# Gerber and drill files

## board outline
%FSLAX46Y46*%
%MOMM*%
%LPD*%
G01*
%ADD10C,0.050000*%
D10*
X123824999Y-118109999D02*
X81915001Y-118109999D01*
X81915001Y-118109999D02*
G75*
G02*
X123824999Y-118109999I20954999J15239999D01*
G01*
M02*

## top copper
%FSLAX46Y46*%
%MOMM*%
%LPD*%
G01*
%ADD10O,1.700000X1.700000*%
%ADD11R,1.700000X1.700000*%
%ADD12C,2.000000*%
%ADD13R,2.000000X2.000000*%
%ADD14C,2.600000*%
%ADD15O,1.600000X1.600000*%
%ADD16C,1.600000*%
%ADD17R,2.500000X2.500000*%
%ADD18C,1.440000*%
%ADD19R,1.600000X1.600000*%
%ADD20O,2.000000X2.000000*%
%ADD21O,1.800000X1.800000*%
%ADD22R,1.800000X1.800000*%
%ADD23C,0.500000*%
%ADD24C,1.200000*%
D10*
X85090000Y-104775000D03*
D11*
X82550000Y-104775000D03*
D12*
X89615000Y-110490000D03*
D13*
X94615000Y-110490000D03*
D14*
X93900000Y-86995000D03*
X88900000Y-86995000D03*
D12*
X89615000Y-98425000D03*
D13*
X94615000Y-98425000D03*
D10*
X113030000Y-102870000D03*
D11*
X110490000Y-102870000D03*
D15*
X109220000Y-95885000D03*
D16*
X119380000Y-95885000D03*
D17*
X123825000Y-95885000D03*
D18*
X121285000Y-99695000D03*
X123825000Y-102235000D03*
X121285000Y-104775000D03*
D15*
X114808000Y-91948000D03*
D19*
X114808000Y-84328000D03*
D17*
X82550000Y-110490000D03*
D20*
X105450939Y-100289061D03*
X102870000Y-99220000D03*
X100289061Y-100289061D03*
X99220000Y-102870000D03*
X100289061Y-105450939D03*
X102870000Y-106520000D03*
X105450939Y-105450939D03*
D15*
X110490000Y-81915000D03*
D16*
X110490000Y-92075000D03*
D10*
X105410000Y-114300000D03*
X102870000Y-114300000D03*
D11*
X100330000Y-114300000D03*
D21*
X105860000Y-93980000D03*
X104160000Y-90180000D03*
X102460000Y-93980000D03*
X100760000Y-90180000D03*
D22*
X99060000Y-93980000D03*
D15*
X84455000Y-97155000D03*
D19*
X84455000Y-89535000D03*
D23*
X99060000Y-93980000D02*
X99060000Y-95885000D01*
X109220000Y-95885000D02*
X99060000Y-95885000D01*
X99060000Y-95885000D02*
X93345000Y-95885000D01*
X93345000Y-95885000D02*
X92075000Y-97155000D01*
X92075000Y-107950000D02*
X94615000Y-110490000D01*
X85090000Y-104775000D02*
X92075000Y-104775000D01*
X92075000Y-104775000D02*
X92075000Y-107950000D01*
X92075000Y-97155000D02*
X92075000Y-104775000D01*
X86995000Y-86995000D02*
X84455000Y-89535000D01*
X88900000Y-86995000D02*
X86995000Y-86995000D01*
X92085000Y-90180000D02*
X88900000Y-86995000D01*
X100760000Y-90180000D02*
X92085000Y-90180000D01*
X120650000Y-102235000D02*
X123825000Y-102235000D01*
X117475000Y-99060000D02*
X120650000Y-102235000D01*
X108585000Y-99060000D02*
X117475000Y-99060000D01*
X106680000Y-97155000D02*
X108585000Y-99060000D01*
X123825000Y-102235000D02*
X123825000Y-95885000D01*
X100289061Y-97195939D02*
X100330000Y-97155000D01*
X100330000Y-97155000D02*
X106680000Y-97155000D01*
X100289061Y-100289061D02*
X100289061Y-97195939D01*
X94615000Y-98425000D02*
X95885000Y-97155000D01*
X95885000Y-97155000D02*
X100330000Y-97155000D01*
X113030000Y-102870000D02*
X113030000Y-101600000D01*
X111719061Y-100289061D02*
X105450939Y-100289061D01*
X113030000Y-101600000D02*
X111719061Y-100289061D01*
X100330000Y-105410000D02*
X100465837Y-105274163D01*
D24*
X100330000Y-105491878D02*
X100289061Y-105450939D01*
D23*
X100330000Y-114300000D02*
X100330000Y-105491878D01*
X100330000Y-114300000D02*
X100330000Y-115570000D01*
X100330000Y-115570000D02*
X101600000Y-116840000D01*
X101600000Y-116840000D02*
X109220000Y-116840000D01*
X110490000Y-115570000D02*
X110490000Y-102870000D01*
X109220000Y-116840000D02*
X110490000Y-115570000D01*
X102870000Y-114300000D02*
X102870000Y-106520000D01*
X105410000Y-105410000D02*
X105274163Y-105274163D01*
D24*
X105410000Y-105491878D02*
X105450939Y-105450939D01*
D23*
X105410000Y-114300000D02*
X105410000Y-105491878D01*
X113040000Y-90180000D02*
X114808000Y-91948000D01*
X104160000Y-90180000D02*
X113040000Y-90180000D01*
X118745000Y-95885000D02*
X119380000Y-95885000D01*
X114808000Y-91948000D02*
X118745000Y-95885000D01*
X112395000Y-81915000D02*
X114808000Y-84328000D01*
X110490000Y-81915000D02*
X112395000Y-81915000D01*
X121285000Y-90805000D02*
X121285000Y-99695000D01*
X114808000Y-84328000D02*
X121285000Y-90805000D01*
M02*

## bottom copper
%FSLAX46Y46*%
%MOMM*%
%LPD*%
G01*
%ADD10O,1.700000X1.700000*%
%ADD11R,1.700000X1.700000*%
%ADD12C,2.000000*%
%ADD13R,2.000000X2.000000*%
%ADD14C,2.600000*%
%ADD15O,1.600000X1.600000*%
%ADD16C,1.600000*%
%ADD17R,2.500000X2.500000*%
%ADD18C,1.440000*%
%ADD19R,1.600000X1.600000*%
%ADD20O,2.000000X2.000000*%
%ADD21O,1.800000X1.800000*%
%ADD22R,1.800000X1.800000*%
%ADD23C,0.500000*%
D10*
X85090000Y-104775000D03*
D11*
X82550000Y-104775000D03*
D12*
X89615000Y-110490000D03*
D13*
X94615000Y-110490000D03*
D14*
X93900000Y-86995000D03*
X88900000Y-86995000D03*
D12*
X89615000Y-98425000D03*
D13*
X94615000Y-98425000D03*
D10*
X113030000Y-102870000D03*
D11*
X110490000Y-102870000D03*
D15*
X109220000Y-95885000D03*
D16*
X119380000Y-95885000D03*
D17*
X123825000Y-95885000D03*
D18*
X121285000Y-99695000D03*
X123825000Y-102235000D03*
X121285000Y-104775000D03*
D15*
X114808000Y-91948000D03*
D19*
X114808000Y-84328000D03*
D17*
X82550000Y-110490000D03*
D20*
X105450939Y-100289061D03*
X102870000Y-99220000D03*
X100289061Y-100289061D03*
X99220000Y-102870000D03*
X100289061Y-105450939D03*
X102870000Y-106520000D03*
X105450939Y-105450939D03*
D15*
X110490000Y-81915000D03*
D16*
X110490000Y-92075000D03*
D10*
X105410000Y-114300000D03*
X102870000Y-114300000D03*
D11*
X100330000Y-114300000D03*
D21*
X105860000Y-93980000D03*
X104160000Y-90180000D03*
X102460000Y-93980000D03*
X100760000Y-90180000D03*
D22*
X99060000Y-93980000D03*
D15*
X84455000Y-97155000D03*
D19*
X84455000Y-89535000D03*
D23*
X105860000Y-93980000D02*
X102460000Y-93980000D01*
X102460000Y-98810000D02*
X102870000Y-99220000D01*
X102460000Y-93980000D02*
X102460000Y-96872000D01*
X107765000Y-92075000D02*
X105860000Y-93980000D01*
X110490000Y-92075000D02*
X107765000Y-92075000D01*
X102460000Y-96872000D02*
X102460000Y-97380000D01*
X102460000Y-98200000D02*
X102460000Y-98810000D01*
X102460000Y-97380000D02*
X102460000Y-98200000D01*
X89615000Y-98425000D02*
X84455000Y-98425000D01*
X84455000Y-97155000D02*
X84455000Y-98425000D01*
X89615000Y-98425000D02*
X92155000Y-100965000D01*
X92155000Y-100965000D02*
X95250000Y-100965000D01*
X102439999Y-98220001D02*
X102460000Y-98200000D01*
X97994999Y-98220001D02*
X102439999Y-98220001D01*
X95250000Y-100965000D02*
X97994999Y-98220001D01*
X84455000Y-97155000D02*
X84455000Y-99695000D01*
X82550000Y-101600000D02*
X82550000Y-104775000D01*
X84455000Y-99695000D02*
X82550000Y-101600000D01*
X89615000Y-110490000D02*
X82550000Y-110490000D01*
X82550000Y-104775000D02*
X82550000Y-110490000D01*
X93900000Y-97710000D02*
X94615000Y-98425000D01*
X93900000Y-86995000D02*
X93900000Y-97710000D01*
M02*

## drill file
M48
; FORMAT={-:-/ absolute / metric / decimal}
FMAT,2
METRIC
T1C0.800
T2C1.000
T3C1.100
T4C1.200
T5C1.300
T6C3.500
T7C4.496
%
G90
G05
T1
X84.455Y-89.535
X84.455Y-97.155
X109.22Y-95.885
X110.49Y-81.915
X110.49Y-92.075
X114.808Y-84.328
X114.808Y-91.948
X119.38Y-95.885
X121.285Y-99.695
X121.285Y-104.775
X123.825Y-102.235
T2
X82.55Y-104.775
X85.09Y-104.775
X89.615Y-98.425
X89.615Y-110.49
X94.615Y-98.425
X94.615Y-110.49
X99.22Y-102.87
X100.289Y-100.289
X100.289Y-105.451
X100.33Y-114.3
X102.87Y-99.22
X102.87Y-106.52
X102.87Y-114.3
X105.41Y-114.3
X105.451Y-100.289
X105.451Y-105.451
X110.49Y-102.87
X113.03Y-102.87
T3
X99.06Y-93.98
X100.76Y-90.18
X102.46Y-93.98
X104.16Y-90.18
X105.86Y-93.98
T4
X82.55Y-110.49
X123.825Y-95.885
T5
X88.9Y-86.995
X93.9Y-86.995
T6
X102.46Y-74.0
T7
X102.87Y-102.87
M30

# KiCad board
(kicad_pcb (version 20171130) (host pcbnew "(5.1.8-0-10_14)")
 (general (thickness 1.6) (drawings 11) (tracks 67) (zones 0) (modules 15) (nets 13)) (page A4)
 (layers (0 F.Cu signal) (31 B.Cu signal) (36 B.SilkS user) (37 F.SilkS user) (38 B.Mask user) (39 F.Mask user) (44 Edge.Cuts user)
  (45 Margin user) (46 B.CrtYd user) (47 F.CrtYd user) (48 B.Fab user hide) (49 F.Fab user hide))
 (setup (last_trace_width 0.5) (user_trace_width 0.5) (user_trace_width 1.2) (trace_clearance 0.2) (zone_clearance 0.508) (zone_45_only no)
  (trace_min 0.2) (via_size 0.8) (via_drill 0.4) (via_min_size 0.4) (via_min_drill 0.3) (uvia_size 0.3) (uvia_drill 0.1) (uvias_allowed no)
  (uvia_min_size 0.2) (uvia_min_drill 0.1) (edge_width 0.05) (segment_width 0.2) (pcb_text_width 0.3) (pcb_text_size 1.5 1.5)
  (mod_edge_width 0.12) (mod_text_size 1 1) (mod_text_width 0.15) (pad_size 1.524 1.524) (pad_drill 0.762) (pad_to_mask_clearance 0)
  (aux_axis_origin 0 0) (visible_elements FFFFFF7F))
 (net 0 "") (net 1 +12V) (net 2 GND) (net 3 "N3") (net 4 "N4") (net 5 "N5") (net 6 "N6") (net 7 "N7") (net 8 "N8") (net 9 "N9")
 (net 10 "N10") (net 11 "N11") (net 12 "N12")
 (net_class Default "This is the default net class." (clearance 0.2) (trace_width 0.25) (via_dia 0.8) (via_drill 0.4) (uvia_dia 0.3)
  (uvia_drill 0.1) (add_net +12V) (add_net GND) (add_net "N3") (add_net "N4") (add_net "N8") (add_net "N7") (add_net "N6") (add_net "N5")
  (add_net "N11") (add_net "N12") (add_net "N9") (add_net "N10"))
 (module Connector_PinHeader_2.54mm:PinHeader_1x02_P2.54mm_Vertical (layer F.Cu) (at 82.55 104.775 90)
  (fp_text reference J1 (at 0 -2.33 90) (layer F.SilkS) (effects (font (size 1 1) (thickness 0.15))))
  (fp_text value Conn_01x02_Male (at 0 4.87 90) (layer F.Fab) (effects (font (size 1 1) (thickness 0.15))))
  (pad 2 thru_hole oval (at 0 2.54 90) (size 1.7 1.7) (drill 1) (layers *.Cu *.Mask) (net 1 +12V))
  (pad 1 thru_hole rect (at 0 0 90) (size 1.7 1.7) (drill 1) (layers *.Cu *.Mask) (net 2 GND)))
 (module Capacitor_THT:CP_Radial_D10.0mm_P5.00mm (layer F.Cu) (at 94.615 110.49 180)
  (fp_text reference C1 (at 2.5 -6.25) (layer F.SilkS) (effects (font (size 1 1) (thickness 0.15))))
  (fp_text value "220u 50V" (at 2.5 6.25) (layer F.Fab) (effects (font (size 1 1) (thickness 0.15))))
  (pad 2 thru_hole circle (at 5 0 180) (size 2 2) (drill 1) (layers *.Cu *.Mask) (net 2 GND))
  (pad 1 thru_hole rect (at 0 0 180) (size 2 2) (drill 1) (layers *.Cu *.Mask) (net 1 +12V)))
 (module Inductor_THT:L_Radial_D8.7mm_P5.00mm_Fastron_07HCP (layer F.Cu) (at 88.9 86.995)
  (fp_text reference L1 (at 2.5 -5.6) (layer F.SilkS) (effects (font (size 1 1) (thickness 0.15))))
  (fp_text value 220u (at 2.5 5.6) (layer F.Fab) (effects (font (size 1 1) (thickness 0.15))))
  (pad 2 thru_hole circle (at 5 0) (size 2.6 2.6) (drill 1.3) (layers *.Cu *.Mask) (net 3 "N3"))
  (pad 1 thru_hole circle (at 0 0) (size 2.6 2.6) (drill 1.3) (layers *.Cu *.Mask) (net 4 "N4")))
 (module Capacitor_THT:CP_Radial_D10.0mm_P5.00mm (layer F.Cu) (at 94.615 98.425 180)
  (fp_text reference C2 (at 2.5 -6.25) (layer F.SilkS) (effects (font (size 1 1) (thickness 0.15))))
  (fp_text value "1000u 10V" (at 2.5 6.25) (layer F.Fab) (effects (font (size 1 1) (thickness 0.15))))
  (pad 2 thru_hole circle (at 5 0 180) (size 2 2) (drill 1) (layers *.Cu *.Mask) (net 2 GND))
  (pad 1 thru_hole rect (at 0 0 180) (size 2 2) (drill 1) (layers *.Cu *.Mask) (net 3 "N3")))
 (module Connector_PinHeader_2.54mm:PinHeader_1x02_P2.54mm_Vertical (layer F.Cu) (at 110.49 102.87 90)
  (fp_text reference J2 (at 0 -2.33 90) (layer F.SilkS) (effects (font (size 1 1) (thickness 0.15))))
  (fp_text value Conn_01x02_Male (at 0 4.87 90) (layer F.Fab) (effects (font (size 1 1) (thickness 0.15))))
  (pad 2 thru_hole oval (at 0 2.54 90) (size 1.7 1.7) (drill 1) (layers *.Cu *.Mask) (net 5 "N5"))
  (pad 1 thru_hole rect (at 0 0 90) (size 1.7 1.7) (drill 1) (layers *.Cu *.Mask) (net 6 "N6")))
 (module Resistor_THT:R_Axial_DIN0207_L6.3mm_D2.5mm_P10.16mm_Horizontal (layer F.Cu) (at 119.38 95.885 180)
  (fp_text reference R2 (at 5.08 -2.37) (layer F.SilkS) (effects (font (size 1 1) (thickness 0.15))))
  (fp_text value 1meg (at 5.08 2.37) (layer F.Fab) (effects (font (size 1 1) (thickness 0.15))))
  (pad 2 thru_hole oval (at 10.16 0 180) (size 1.6 1.6) (drill 0.8) (layers *.Cu *.Mask) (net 1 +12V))
  (pad 1 thru_hole circle (at 0 0 180) (size 1.6 1.6) (drill 0.8) (layers *.Cu *.Mask) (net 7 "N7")))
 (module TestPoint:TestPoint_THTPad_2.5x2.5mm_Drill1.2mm (layer F.Cu) (at 123.825 95.885)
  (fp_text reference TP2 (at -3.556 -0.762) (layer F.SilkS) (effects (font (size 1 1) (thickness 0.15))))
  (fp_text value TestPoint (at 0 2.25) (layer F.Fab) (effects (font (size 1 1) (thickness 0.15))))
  (pad 1 thru_hole rect (at 0 0) (size 2.5 2.5) (drill 1.2) (layers *.Cu *.Mask) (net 3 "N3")))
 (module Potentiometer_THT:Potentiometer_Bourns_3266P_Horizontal (layer F.Cu) (at 121.285 104.775 180)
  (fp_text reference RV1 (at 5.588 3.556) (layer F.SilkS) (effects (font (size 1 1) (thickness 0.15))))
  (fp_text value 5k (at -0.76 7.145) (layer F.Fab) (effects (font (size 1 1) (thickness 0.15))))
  (pad 3 thru_hole circle (at 0 5.08 180) (size 1.44 1.44) (drill 0.8) (layers *.Cu *.Mask) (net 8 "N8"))
  (pad 2 thru_hole circle (at -2.54 2.54 180) (size 1.44 1.44) (drill 0.8) (layers *.Cu *.Mask) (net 3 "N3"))
  (pad 1 thru_hole circle (at 0 0 180) (size 1.44 1.44) (drill 0.8) (layers *.Cu *.Mask) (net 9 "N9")))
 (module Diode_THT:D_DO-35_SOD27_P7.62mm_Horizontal (layer F.Cu) (at 114.808 84.328 270)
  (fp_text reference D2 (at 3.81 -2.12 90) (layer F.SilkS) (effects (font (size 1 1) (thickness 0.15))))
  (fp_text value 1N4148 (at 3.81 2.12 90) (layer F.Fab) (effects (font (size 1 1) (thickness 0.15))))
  (pad 2 thru_hole oval (at 7.62 0 270) (size 1.6 1.6) (drill 0.8) (layers *.Cu *.Mask) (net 7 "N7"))
  (pad 1 thru_hole rect (at 0 0 270) (size 1.6 1.6) (drill 0.8) (layers *.Cu *.Mask) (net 8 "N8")))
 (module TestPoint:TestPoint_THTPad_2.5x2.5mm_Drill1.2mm (layer F.Cu) (at 82.55 110.49)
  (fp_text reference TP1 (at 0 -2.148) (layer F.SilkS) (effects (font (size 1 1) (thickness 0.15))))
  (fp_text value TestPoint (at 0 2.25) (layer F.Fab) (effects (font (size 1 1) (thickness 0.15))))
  (pad 1 thru_hole rect (at 0 0) (size 2.5 2.5) (drill 1.2) (layers *.Cu *.Mask) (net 2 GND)))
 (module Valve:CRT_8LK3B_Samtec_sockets (layer F.Cu) (at 102.87 102.87)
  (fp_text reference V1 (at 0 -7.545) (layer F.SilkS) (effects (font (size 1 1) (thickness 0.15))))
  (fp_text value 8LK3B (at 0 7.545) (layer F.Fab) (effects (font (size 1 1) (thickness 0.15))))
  (pad "" np_thru_hole circle (at 0 0) (size 4.4958 4.4958) (drill 4.4958) (layers *.Mask F.Cu))
  (pad 7 thru_hole oval (at 2.580939 -2.580939) (size 2 2) (drill 1) (layers *.Cu *.Mask) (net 5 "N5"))
  (pad 6 thru_hole oval (at 0 -3.65) (size 2 2) (drill 1) (layers *.Cu *.Mask) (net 2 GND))
  (pad 5 thru_hole oval (at -2.580939 -2.580939) (size 2 2) (drill 1) (layers *.Cu *.Mask) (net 3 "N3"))
  (pad 4 thru_hole oval (at -3.65 0) (size 2 2) (drill 1) (layers *.Cu *.Mask) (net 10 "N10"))
  (pad 3 thru_hole oval (at -2.580939 2.580939) (size 2 2) (drill 1) (layers *.Cu *.Mask) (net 6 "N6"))
  (pad 2 thru_hole oval (at 0 3.65) (size 2 2) (drill 1) (layers *.Cu *.Mask) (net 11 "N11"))
  (pad 1 thru_hole oval (at 2.580939 2.580939) (size 2 2) (drill 1) (layers *.Cu *.Mask) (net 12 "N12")))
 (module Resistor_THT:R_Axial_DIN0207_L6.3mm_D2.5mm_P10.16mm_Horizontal (layer F.Cu) (at 110.49 92.075 90)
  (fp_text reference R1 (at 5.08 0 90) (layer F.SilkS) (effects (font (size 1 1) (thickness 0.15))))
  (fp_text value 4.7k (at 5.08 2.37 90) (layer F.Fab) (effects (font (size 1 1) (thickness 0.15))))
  (pad 2 thru_hole oval (at 10.16 0 90) (size 1.6 1.6) (drill 0.8) (layers *.Cu *.Mask) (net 8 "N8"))
  (pad 1 thru_hole circle (at 0 0 90) (size 1.6 1.6) (drill 0.8) (layers *.Cu *.Mask) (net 2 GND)))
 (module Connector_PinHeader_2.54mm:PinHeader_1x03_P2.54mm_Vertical (layer F.Cu) (at 100.33 114.3 90)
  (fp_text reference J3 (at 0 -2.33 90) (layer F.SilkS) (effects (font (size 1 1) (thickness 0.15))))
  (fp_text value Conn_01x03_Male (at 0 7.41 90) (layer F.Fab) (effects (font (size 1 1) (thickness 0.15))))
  (pad 3 thru_hole oval (at 0 5.08 90) (size 1.7 1.7) (drill 1) (layers *.Cu *.Mask) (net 12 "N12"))
  (pad 2 thru_hole oval (at 0 2.54 90) (size 1.7 1.7) (drill 1) (layers *.Cu *.Mask) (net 11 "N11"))
  (pad 1 thru_hole rect (at 0 0 90) (size 1.7 1.7) (drill 1) (layers *.Cu *.Mask) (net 6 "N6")))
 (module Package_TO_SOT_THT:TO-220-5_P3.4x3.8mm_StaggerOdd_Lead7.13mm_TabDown (layer F.Cu) (at 99.06 93.98)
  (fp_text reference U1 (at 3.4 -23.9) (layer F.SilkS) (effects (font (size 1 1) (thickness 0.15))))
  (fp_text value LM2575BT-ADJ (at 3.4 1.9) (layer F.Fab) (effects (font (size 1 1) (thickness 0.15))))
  (pad 5 thru_hole oval (at 6.8 0) (size 1.8 1.8) (drill 1.1) (layers *.Cu *.Mask) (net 2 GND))
  (pad 4 thru_hole oval (at 5.1 -3.8) (size 1.8 1.8) (drill 1.1) (layers *.Cu *.Mask) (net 7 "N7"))
  (pad 3 thru_hole oval (at 3.4 0) (size 1.8 1.8) (drill 1.1) (layers *.Cu *.Mask) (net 2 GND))
  (pad 2 thru_hole oval (at 1.7 -3.8) (size 1.8 1.8) (drill 1.1) (layers *.Cu *.Mask) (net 4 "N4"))
  (pad 1 thru_hole rect (at 0 0) (size 1.8 1.8) (drill 1.1) (layers *.Cu *.Mask) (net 1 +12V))
  (pad "" np_thru_hole oval (at 3.4 -19.98) (size 3.5 3.5) (drill 3.5) (layers *.Cu *.Mask)))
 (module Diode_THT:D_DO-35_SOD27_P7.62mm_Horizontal (layer F.Cu) (at 84.455 89.535 270)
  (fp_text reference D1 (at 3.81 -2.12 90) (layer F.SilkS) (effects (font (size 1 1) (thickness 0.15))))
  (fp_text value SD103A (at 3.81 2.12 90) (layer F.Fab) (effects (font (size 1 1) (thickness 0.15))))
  (pad 2 thru_hole oval (at 7.62 0 270) (size 1.6 1.6) (drill 0.8) (layers *.Cu *.Mask) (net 2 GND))
  (pad 1 thru_hole rect (at 0 0 270) (size 1.6 1.6) (drill 0.8) (layers *.Cu *.Mask) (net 4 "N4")))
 (gr_line (start 123.824999 118.109999) (end 81.915001 118.109999) (layer Edge.Cuts) (width 0.05))
 (gr_arc (start 102.87 102.87) (end 123.824999 118.109999) (angle -252.0547468) (layer Edge.Cuts) (width 0.05))
 (segment (start 105.86 93.98) (end 102.46 93.98) (width 0.5) (layer B.Cu) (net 2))
 (segment (start 102.46 98.81) (end 102.87 99.22) (width 0.5) (layer B.Cu) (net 2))
 (segment (start 102.46 93.98) (end 102.46 96.872) (width 0.5) (layer B.Cu) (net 2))
 (segment (start 107.765 92.075) (end 105.86 93.98) (width 0.5) (layer B.Cu) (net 2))
 (segment (start 110.49 92.075) (end 107.765 92.075) (width 0.5) (layer B.Cu) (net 2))
 (segment (start 102.46 96.872) (end 102.46 97.38) (width 0.5) (layer B.Cu) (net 2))
 (segment (start 102.46 98.2) (end 102.46 98.81) (width 0.5) (layer B.Cu) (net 2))
 (segment (start 102.46 97.38) (end 102.46 98.2) (width 0.5) (layer B.Cu) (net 2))
 (segment (start 89.615 98.425) (end 84.455 98.425) (width 0.5) (layer B.Cu) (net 2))
 (segment (start 84.455 97.155) (end 84.455 98.425) (width 0.5) (layer B.Cu) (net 2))
 (segment (start 89.615 98.425) (end 92.155 100.965) (width 0.5) (layer B.Cu) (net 2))
 (segment (start 92.155 100.965) (end 95.25 100.965) (width 0.5) (layer B.Cu) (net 2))
 (segment (start 102.439999 98.220001) (end 102.46 98.2) (width 0.5) (layer B.Cu) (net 2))
 (segment (start 97.994999 98.220001) (end 102.439999 98.220001) (width 0.5) (layer B.Cu) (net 2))
 (segment (start 95.25 100.965) (end 97.994999 98.220001) (width 0.5) (layer B.Cu) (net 2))
 (segment (start 84.455 97.155) (end 84.455 99.695) (width 0.5) (layer B.Cu) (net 2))
 (segment (start 82.55 101.6) (end 82.55 104.775) (width 0.5) (layer B.Cu) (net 2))
 (segment (start 84.455 99.695) (end 82.55 101.6) (width 0.5) (layer B.Cu) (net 2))
 (segment (start 89.615 110.49) (end 82.55 110.49) (width 0.5) (layer B.Cu) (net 2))
 (segment (start 82.55 104.775) (end 82.55 110.49) (width 0.5) (layer B.Cu) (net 2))
 (segment (start 99.06 93.98) (end 99.06 95.885) (width 0.5) (layer F.Cu) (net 1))
 (segment (start 109.22 95.885) (end 99.06 95.885) (width 0.5) (layer F.Cu) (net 1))
 (segment (start 99.06 95.885) (end 93.345 95.885) (width 0.5) (layer F.Cu) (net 1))
 (segment (start 93.345 95.885) (end 92.075 97.155) (width 0.5) (layer F.Cu) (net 1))
 (segment (start 92.075 107.95) (end 94.615 110.49) (width 0.5) (layer F.Cu) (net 1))
 (segment (start 85.09 104.775) (end 92.075 104.775) (width 0.5) (layer F.Cu) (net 1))
 (segment (start 92.075 104.775) (end 92.075 107.95) (width 0.5) (layer F.Cu) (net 1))
 (segment (start 92.075 97.155) (end 92.075 104.775) (width 0.5) (layer F.Cu) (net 1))
 (segment (start 86.995 86.995) (end 84.455 89.535) (width 0.5) (layer F.Cu) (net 4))
 (segment (start 88.9 86.995) (end 86.995 86.995) (width 0.5) (layer F.Cu) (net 4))
 (segment (start 92.085 90.18) (end 88.9 86.995) (width 0.5) (layer F.Cu) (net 4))
 (segment (start 100.76 90.18) (end 92.085 90.18) (width 0.5) (layer F.Cu) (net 4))
 (segment (start 120.65 102.235) (end 123.825 102.235) (width 0.5) (layer F.Cu) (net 3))
 (segment (start 117.475 99.06) (end 120.65 102.235) (width 0.5) (layer F.Cu) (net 3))
 (segment (start 108.585 99.06) (end 117.475 99.06) (width 0.5) (layer F.Cu) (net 3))
 (segment (start 106.68 97.155) (end 108.585 99.06) (width 0.5) (layer F.Cu) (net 3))
 (segment (start 123.825 102.235) (end 123.825 95.885) (width 0.5) (layer F.Cu) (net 3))
 (segment (start 100.289061 97.195939) (end 100.33 97.155) (width 0.5) (layer F.Cu) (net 3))
 (segment (start 100.33 97.155) (end 106.68 97.155) (width 0.5) (layer F.Cu) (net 3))
 (segment (start 100.289061 100.289061) (end 100.289061 97.195939) (width 0.5) (layer F.Cu) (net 3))
 (segment (start 94.615 98.425) (end 95.885 97.155) (width 0.5) (layer F.Cu) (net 3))
 (segment (start 95.885 97.155) (end 100.33 97.155) (width 0.5) (layer F.Cu) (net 3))
 (segment (start 93.9 97.71) (end 94.615 98.425) (width 0.5) (layer B.Cu) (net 3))
 (segment (start 93.9 86.995) (end 93.9 97.71) (width 0.5) (layer B.Cu) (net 3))
 (segment (start 113.03 102.87) (end 113.03 101.6) (width 0.5) (layer F.Cu) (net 5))
 (segment (start 111.719061 100.289061) (end 105.450939 100.289061) (width 0.5) (layer F.Cu) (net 5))
 (segment (start 113.03 101.6) (end 111.719061 100.289061) (width 0.5) (layer F.Cu) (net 5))
 (segment (start 100.33 105.41) (end 100.465837 105.274163) (width 0.5) (layer F.Cu) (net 6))
 (segment (start 100.33 105.491878) (end 100.289061 105.450939) (width 1.2) (layer F.Cu) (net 6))
 (segment (start 100.33 114.3) (end 100.33 105.491878) (width 0.5) (layer F.Cu) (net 6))
 (segment (start 100.33 114.3) (end 100.33 115.57) (width 0.5) (layer F.Cu) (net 6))
 (segment (start 100.33 115.57) (end 101.6 116.84) (width 0.5) (layer F.Cu) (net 6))
 (segment (start 101.6 116.84) (end 109.22 116.84) (width 0.5) (layer F.Cu) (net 6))
 (segment (start 110.49 115.57) (end 110.49 102.87) (width 0.5) (layer F.Cu) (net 6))
 (segment (start 109.22 116.84) (end 110.49 115.57) (width 0.5) (layer F.Cu) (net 6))
 (segment (start 102.87 114.3) (end 102.87 106.52) (width 0.5) (layer F.Cu) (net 11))
 (segment (start 105.41 105.41) (end 105.274163 105.274163) (width 0.5) (layer F.Cu) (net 12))
 (segment (start 105.41 105.491878) (end 105.450939 105.450939) (width 1.2) (layer F.Cu) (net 12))
 (segment (start 105.41 114.3) (end 105.41 105.491878) (width 0.5) (layer F.Cu) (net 12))
 (segment (start 113.04 90.18) (end 114.808 91.948) (width 0.5) (layer F.Cu) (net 7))
 (segment (start 104.16 90.18) (end 113.04 90.18) (width 0.5) (layer F.Cu) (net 7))
 (segment (start 118.745 95.885) (end 119.38 95.885) (width 0.5) (layer F.Cu) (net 7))
 (segment (start 114.808 91.948) (end 118.745 95.885) (width 0.5) (layer F.Cu) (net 7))
 (segment (start 112.395 81.915) (end 114.808 84.328) (width 0.5) (layer F.Cu) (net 8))
 (segment (start 110.49 81.915) (end 112.395 81.915) (width 0.5) (layer F.Cu) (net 8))
 (segment (start 121.285 90.805) (end 121.285 99.695) (width 0.5) (layer F.Cu) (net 8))
 (segment (start 114.808 84.328) (end 121.285 90.805) (width 0.5) (layer F.Cu) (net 8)))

